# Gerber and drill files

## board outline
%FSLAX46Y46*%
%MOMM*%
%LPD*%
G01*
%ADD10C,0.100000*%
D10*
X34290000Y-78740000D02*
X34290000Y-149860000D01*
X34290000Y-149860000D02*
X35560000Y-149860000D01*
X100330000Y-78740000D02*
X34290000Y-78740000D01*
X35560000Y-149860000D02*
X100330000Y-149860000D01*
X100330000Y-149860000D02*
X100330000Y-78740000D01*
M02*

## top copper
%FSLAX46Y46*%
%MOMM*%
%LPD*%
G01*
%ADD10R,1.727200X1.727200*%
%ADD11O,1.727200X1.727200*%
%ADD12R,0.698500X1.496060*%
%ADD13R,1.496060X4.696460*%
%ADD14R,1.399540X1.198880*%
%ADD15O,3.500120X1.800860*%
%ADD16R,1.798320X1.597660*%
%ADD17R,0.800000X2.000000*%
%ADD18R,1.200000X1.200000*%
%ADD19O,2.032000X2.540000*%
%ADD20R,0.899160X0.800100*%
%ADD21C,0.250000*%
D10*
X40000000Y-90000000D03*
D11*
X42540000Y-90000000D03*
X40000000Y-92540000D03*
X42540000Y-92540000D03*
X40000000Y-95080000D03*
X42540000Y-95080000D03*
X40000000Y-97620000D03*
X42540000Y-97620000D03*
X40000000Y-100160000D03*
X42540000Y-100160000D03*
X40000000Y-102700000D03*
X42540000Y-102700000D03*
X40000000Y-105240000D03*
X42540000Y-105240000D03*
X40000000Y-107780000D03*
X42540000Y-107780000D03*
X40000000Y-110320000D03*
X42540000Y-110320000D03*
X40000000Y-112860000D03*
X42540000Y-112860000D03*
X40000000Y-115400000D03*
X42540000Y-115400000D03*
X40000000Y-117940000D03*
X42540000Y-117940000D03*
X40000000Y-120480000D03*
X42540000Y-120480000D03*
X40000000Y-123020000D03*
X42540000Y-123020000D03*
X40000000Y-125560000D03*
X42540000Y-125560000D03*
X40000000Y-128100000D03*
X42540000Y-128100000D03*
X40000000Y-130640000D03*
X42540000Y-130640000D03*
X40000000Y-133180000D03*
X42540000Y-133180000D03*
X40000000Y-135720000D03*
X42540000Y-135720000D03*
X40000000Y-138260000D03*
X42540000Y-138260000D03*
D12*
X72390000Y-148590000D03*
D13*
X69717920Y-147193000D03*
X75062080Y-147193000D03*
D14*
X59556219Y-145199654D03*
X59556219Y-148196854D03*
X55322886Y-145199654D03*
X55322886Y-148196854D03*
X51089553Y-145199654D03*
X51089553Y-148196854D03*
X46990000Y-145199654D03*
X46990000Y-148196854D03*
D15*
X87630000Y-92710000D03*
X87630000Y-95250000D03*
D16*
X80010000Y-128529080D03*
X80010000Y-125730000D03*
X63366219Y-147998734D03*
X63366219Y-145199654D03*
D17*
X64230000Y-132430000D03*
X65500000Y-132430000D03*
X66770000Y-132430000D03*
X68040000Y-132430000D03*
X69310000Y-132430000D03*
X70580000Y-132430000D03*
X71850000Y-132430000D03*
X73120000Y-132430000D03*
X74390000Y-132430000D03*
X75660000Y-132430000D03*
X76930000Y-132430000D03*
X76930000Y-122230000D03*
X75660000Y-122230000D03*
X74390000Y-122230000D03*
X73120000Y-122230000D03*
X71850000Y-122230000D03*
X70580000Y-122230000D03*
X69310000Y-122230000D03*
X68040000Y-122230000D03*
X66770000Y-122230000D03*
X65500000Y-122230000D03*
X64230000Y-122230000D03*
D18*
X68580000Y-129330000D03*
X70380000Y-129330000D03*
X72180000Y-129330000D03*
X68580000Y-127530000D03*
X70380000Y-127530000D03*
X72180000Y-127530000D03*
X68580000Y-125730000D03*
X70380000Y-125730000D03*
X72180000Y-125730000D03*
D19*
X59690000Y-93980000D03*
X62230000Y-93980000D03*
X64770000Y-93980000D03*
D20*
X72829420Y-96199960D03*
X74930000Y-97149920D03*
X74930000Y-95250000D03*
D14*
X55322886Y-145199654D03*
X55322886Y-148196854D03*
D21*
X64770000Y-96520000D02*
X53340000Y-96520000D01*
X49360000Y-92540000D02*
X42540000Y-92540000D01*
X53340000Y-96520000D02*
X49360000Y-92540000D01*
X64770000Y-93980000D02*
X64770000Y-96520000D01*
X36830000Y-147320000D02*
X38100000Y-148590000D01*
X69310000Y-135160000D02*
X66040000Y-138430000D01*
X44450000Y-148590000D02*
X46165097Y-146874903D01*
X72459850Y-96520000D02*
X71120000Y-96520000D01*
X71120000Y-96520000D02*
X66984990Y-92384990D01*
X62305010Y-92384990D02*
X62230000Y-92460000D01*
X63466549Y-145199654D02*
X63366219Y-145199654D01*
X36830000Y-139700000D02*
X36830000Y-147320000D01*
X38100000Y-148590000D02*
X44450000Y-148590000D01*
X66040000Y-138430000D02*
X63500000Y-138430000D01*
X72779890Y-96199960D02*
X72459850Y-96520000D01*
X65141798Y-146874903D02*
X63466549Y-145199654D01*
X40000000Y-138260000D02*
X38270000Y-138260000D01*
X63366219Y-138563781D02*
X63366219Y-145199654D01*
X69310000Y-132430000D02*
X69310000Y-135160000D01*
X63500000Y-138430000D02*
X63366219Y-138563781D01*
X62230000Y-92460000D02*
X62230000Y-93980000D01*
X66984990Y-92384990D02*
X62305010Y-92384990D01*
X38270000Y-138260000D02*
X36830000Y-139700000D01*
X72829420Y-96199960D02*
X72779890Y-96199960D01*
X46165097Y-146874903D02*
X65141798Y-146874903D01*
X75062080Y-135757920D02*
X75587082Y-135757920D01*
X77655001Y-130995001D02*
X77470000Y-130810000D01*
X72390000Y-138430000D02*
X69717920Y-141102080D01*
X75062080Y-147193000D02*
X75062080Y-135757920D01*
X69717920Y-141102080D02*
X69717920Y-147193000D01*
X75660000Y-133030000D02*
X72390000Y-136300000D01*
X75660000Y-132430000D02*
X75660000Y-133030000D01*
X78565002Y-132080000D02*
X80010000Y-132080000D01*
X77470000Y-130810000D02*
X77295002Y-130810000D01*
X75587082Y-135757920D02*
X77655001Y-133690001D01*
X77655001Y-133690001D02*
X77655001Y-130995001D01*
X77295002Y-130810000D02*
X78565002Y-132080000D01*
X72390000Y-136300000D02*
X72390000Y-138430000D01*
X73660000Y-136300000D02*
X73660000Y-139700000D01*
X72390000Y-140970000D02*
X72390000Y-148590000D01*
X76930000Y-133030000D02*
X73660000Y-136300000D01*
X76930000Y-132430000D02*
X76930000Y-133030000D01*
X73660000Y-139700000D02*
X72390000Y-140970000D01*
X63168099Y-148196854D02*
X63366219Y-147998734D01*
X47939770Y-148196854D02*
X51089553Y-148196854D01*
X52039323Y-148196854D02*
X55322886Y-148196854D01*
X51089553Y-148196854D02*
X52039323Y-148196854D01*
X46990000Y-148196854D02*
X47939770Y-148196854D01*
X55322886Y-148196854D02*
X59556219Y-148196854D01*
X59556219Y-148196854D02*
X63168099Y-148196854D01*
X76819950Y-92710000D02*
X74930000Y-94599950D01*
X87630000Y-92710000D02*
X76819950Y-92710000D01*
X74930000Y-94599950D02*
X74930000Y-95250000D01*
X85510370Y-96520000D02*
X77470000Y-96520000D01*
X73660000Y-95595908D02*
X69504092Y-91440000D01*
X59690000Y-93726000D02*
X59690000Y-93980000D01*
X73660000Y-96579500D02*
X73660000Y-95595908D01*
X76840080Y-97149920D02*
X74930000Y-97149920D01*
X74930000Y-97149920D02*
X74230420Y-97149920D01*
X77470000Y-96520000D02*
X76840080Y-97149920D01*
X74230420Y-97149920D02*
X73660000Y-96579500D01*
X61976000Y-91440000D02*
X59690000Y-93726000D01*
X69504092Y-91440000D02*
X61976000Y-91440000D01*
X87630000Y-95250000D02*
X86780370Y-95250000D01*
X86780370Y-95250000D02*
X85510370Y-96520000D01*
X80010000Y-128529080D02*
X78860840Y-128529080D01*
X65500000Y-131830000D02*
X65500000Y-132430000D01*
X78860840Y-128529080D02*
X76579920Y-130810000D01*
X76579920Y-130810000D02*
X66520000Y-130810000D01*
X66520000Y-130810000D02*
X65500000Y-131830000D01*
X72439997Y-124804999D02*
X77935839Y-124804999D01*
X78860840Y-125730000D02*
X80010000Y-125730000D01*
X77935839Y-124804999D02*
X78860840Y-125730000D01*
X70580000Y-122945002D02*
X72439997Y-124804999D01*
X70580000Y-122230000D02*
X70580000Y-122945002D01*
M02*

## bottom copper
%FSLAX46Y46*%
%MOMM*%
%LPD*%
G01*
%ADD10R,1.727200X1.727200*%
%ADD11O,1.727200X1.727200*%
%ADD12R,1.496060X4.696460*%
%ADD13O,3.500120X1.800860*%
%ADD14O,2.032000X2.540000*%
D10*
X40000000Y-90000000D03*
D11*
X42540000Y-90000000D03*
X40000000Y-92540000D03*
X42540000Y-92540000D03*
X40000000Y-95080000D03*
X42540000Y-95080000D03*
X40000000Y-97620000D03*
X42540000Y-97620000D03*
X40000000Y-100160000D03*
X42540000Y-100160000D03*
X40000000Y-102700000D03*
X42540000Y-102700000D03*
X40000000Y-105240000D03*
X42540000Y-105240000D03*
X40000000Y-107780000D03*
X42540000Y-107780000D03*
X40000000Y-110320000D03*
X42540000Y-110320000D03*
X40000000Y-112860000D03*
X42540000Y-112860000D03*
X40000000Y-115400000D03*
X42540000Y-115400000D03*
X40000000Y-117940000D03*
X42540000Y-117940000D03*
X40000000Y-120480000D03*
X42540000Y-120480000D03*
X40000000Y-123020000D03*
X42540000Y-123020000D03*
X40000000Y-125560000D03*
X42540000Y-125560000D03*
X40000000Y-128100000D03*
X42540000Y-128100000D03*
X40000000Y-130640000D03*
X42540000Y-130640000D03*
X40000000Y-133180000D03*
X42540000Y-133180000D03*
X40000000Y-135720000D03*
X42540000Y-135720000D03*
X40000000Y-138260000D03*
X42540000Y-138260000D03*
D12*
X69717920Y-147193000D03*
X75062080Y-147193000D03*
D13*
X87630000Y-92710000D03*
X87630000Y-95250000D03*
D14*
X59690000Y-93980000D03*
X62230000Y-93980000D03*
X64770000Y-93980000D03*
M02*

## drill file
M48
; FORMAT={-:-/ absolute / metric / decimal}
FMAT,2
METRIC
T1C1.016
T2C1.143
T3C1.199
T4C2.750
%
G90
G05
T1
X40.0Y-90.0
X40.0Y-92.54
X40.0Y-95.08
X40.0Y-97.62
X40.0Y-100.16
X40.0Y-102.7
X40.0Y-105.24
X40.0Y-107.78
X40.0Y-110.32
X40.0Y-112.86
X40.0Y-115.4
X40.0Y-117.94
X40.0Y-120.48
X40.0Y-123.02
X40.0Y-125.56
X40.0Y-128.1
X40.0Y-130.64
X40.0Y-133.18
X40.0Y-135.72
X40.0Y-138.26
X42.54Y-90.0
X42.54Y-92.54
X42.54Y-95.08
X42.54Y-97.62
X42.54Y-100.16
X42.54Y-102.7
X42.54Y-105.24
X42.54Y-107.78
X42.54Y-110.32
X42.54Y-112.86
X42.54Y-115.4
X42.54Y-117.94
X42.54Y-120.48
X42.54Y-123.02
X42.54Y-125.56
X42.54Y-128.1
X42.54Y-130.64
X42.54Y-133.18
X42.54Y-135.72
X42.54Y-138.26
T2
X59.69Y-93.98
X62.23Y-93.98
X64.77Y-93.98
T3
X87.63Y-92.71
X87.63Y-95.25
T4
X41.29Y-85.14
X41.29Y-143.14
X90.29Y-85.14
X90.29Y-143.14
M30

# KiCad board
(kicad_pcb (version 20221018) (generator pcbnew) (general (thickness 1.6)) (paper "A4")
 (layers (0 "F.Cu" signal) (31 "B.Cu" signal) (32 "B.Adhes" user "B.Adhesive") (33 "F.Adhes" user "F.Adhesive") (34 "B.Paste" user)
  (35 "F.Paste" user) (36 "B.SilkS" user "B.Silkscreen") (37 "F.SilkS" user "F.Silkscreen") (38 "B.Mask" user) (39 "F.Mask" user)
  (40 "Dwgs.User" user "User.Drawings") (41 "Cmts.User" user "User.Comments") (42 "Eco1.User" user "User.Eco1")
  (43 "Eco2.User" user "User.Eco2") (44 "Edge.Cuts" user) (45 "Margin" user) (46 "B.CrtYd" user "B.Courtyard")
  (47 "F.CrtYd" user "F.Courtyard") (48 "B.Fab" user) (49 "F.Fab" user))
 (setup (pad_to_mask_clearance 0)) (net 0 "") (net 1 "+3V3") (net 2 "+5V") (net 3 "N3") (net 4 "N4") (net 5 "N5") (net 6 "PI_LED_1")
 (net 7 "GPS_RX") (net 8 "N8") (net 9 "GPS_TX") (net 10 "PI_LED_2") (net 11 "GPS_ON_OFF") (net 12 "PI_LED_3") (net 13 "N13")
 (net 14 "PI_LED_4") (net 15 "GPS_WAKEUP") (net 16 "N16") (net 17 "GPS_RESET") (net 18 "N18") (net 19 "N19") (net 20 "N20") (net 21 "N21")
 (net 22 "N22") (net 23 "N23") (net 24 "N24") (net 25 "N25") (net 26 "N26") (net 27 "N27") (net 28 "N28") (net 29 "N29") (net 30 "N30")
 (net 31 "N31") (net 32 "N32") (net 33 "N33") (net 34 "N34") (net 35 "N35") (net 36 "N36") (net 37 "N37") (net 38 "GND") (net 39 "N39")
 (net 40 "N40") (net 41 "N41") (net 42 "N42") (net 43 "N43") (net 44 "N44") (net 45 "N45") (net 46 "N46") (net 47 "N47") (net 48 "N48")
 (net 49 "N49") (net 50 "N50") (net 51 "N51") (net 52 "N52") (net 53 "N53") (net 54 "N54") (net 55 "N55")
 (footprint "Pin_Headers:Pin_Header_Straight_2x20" (layer "F.Cu") (at 40 90)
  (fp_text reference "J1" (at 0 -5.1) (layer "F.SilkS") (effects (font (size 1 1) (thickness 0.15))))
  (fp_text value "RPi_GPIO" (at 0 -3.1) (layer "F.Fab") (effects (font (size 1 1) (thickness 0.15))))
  (pad "1" thru_hole rect (at 0 0) (size 1.7272 1.7272) (drill 1.016) (layers "*.Cu" "*.Mask" "F.SilkS") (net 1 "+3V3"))
  (pad "2" thru_hole oval (at 2.54 0) (size 1.7272 1.7272) (drill 1.016) (layers "*.Cu" "*.Mask" "F.SilkS") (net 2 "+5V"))
  (pad "3" thru_hole oval (at 0 2.54) (size 1.7272 1.7272) (drill 1.016) (layers "*.Cu" "*.Mask" "F.SilkS") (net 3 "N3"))
  (pad "4" thru_hole oval (at 2.54 2.54) (size 1.7272 1.7272) (drill 1.016) (layers "*.Cu" "*.Mask" "F.SilkS") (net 2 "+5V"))
  (pad "5" thru_hole oval (at 0 5.08) (size 1.7272 1.7272) (drill 1.016) (layers "*.Cu" "*.Mask" "F.SilkS") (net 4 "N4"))
  (pad "6" thru_hole oval (at 2.54 5.08) (size 1.7272 1.7272) (drill 1.016) (layers "*.Cu" "*.Mask" "F.SilkS") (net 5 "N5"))
  (pad "7" thru_hole oval (at 0 7.62) (size 1.7272 1.7272) (drill 1.016) (layers "*.Cu" "*.Mask" "F.SilkS") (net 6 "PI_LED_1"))
  (pad "8" thru_hole oval (at 2.54 7.62) (size 1.7272 1.7272) (drill 1.016) (layers "*.Cu" "*.Mask" "F.SilkS") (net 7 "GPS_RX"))
  (pad "9" thru_hole oval (at 0 10.16) (size 1.7272 1.7272) (drill 1.016) (layers "*.Cu" "*.Mask" "F.SilkS") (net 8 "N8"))
  (pad "10" thru_hole oval (at 2.54 10.16) (size 1.7272 1.7272) (drill 1.016) (layers "*.Cu" "*.Mask" "F.SilkS") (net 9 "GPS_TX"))
  (pad "11" thru_hole oval (at 0 12.7) (size 1.7272 1.7272) (drill 1.016) (layers "*.Cu" "*.Mask" "F.SilkS") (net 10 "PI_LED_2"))
  (pad "12" thru_hole oval (at 2.54 12.7) (size 1.7272 1.7272) (drill 1.016) (layers "*.Cu" "*.Mask" "F.SilkS") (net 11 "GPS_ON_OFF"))
  (pad "13" thru_hole oval (at 0 15.24) (size 1.7272 1.7272) (drill 1.016) (layers "*.Cu" "*.Mask" "F.SilkS") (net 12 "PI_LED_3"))
  (pad "14" thru_hole oval (at 2.54 15.24) (size 1.7272 1.7272) (drill 1.016) (layers "*.Cu" "*.Mask" "F.SilkS") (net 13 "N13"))
  (pad "15" thru_hole oval (at 0 17.78) (size 1.7272 1.7272) (drill 1.016) (layers "*.Cu" "*.Mask" "F.SilkS") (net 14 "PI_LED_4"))
  (pad "16" thru_hole oval (at 2.54 17.78) (size 1.7272 1.7272) (drill 1.016) (layers "*.Cu" "*.Mask" "F.SilkS") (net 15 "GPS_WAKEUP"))
  (pad "17" thru_hole oval (at 0 20.32) (size 1.7272 1.7272) (drill 1.016) (layers "*.Cu" "*.Mask" "F.SilkS") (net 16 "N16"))
  (pad "18" thru_hole oval (at 2.54 20.32) (size 1.7272 1.7272) (drill 1.016) (layers "*.Cu" "*.Mask" "F.SilkS") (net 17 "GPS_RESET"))
  (pad "19" thru_hole oval (at 0 22.86) (size 1.7272 1.7272) (drill 1.016) (layers "*.Cu" "*.Mask" "F.SilkS") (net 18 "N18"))
  (pad "20" thru_hole oval (at 2.54 22.86) (size 1.7272 1.7272) (drill 1.016) (layers "*.Cu" "*.Mask" "F.SilkS") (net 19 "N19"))
  (pad "21" thru_hole oval (at 0 25.4) (size 1.7272 1.7272) (drill 1.016) (layers "*.Cu" "*.Mask" "F.SilkS") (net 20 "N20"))
  (pad "22" thru_hole oval (at 2.54 25.4) (size 1.7272 1.7272) (drill 1.016) (layers "*.Cu" "*.Mask" "F.SilkS") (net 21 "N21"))
  (pad "23" thru_hole oval (at 0 27.94) (size 1.7272 1.7272) (drill 1.016) (layers "*.Cu" "*.Mask" "F.SilkS") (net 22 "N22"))
  (pad "24" thru_hole oval (at 2.54 27.94) (size 1.7272 1.7272) (drill 1.016) (layers "*.Cu" "*.Mask" "F.SilkS") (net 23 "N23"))
  (pad "25" thru_hole oval (at 0 30.48) (size 1.7272 1.7272) (drill 1.016) (layers "*.Cu" "*.Mask" "F.SilkS") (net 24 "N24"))
  (pad "26" thru_hole oval (at 2.54 30.48) (size 1.7272 1.7272) (drill 1.016) (layers "*.Cu" "*.Mask" "F.SilkS") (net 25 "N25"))
  (pad "27" thru_hole oval (at 0 33.02) (size 1.7272 1.7272) (drill 1.016) (layers "*.Cu" "*.Mask" "F.SilkS") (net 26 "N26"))
  (pad "28" thru_hole oval (at 2.54 33.02) (size 1.7272 1.7272) (drill 1.016) (layers "*.Cu" "*.Mask" "F.SilkS") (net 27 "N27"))
  (pad "29" thru_hole oval (at 0 35.56) (size 1.7272 1.7272) (drill 1.016) (layers "*.Cu" "*.Mask" "F.SilkS") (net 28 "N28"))
  (pad "30" thru_hole oval (at 2.54 35.56) (size 1.7272 1.7272) (drill 1.016) (layers "*.Cu" "*.Mask" "F.SilkS") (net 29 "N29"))
  (pad "31" thru_hole oval (at 0 38.1) (size 1.7272 1.7272) (drill 1.016) (layers "*.Cu" "*.Mask" "F.SilkS") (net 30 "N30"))
  (pad "32" thru_hole oval (at 2.54 38.1) (size 1.7272 1.7272) (drill 1.016) (layers "*.Cu" "*.Mask" "F.SilkS") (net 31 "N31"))
  (pad "33" thru_hole oval (at 0 40.64) (size 1.7272 1.7272) (drill 1.016) (layers "*.Cu" "*.Mask" "F.SilkS") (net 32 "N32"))
  (pad "34" thru_hole oval (at 2.54 40.64) (size 1.7272 1.7272) (drill 1.016) (layers "*.Cu" "*.Mask" "F.SilkS") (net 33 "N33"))
  (pad "35" thru_hole oval (at 0 43.18) (size 1.7272 1.7272) (drill 1.016) (layers "*.Cu" "*.Mask" "F.SilkS") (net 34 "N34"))
  (pad "36" thru_hole oval (at 2.54 43.18) (size 1.7272 1.7272) (drill 1.016) (layers "*.Cu" "*.Mask" "F.SilkS") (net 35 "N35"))
  (pad "37" thru_hole oval (at 0 45.72) (size 1.7272 1.7272) (drill 1.016) (layers "*.Cu" "*.Mask" "F.SilkS") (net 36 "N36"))
  (pad "38" thru_hole oval (at 2.54 45.72) (size 1.7272 1.7272) (drill 1.016) (layers "*.Cu" "*.Mask" "F.SilkS") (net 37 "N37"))
  (pad "39" thru_hole oval (at 0 48.26) (size 1.7272 1.7272) (drill 1.016) (layers "*.Cu" "*.Mask" "F.SilkS") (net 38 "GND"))
  (pad "40" thru_hole oval (at 2.54 48.26) (size 1.7272 1.7272) (drill 1.016) (layers "*.Cu" "*.Mask" "F.SilkS") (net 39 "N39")))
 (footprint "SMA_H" (layer "F.Cu") (at 72.39 147.193 -90)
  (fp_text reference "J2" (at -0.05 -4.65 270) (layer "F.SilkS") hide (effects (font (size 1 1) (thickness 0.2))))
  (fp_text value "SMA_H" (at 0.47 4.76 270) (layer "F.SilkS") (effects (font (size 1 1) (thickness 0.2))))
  (pad "1" smd rect (at 1.397 0 270) (size 1.49606 0.6985) (layers "F.Cu" "F.Paste" "F.Mask") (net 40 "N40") (clearance 0.19558))
  (pad "2" smd rect (at 0 2.67208 270) (size 4.69646 1.49606) (layers "F.Cu" "F.Paste" "F.Mask") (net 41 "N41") (clearance 0.19558))
  (pad "3" smd rect (at 0 -2.67208 270) (size 4.69646 1.49606) (layers "F.Cu" "F.Paste" "F.Mask") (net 41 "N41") (clearance 0.19558))
  (pad "4" smd rect (at 0 2.67208 270) (size 4.69646 1.49606) (layers "B.Cu" "B.Paste" "B.Mask") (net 41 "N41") (clearance 0.19558))
  (pad "5" smd rect (at 0 -2.67208 270) (size 4.69646 1.49606) (layers "B.Cu" "B.Paste" "B.Mask") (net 41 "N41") (clearance 0.19558)))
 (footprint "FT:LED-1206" (layer "F.Cu") (at 59.556219 146.698254 -90)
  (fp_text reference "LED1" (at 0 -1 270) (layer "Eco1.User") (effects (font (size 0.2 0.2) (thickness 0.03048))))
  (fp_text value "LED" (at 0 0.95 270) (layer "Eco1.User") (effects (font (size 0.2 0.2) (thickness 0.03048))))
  (pad "A" smd rect (at -1.4986 0 270) (size 1.19888 1.39954) (layers "F.Cu" "F.Paste" "F.Mask") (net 6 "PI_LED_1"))
  (pad "K" smd rect (at 1.4986 0 270) (size 1.19888 1.39954) (layers "F.Cu" "F.Paste" "F.Mask") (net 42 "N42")))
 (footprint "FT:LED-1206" (layer "F.Cu") (at 55.322886 146.698254 -90)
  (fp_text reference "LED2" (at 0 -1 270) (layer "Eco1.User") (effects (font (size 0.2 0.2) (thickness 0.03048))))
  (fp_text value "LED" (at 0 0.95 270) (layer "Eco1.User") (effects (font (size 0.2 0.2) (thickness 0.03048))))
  (pad "A" smd rect (at -1.4986 0 270) (size 1.19888 1.39954) (layers "F.Cu" "F.Paste" "F.Mask") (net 10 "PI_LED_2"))
  (pad "K" smd rect (at 1.4986 0 270) (size 1.19888 1.39954) (layers "F.Cu" "F.Paste" "F.Mask") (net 42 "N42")))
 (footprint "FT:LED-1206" (layer "F.Cu") (at 51.089553 146.698254 -90)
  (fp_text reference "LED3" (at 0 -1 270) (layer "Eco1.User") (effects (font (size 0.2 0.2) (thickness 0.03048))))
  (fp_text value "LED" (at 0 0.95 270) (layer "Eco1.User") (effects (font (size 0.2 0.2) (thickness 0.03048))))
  (pad "A" smd rect (at -1.4986 0 270) (size 1.19888 1.39954) (layers "F.Cu" "F.Paste" "F.Mask") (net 12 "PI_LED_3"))
  (pad "K" smd rect (at 1.4986 0 270) (size 1.19888 1.39954) (layers "F.Cu" "F.Paste" "F.Mask") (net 42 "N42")))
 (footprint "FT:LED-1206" (layer "F.Cu") (at 46.99 146.698254 -90)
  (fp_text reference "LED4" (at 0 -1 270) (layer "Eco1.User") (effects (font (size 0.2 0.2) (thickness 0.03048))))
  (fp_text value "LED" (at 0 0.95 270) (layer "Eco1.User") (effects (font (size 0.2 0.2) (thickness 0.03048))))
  (pad "A" smd rect (at -1.4986 0 270) (size 1.19888 1.39954) (layers "F.Cu" "F.Paste" "F.Mask") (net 14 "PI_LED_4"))
  (pad "K" smd rect (at 1.4986 0 270) (size 1.19888 1.39954) (layers "F.Cu" "F.Paste" "F.Mask") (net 42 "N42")))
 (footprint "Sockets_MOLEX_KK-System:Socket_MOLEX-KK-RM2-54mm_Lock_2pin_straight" (layer "F.Cu") (at 87.63 93.98 -90)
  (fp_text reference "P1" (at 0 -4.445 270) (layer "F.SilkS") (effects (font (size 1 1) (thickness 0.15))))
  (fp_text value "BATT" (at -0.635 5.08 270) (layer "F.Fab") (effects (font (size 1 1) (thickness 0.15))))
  (pad "1" thru_hole oval (at -1.27 0 270) (size 1.80086 3.50012) (drill 1.19888) (layers "*.Cu" "*.Mask" "F.SilkS") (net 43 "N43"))
  (pad "2" thru_hole oval (at 1.27 0 270) (size 1.80086 3.50012) (drill 1.19888) (layers "*.Cu" "*.Mask" "F.SilkS") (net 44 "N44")))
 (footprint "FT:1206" (layer "F.Cu") (at 80.01 127.12954 90)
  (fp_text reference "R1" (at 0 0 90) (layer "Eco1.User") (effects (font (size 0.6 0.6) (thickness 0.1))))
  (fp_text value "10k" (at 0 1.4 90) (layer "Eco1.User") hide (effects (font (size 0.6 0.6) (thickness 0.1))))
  (pad "1" smd rect (at -1.39954 0 90) (size 1.59766 1.79832) (layers "F.Cu" "F.Paste" "F.Mask") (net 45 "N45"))
  (pad "2" smd rect (at 1.39954 0 90) (size 1.59766 1.79832) (layers "F.Cu" "F.Paste" "F.Mask") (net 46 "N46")))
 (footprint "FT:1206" (layer "F.Cu") (at 63.366219 146.599194 90)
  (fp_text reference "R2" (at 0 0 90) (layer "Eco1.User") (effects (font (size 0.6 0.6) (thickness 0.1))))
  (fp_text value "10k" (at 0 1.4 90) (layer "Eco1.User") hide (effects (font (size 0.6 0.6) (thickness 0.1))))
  (pad "1" smd rect (at -1.39954 0 90) (size 1.59766 1.79832) (layers "F.Cu" "F.Paste" "F.Mask") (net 42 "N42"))
  (pad "2" smd rect (at 1.39954 0 90) (size 1.59766 1.79832) (layers "F.Cu" "F.Paste" "F.Mask") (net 38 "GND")))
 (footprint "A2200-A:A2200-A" (layer "F.Cu") (at 70.38 127.53 90)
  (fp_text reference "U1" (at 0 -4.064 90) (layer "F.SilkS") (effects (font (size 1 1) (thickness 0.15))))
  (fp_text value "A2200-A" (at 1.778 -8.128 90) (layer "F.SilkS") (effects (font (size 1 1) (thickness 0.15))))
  (pad "1" smd rect (at -4.9 -6.15 90) (size 2 0.8) (layers "F.Cu" "F.Paste" "F.Mask") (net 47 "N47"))
  (pad "2" smd rect (at -4.9 -4.88 90) (size 2 0.8) (layers "F.Cu" "F.Paste" "F.Mask") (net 45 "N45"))
  (pad "3" smd rect (at -4.9 -3.61 90) (size 2 0.8) (layers "F.Cu" "F.Paste" "F.Mask") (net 9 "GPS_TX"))
  (pad "4" smd rect (at -4.9 -2.34 90) (size 2 0.8) (layers "F.Cu" "F.Paste" "F.Mask") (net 7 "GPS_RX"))
  (pad "5" smd rect (at -4.9 -1.07 90) (size 2 0.8) (layers "F.Cu" "F.Paste" "F.Mask") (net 38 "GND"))
  (pad "6" smd rect (at -4.9 0.2 90) (size 2 0.8) (layers "F.Cu" "F.Paste" "F.Mask") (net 11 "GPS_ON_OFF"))
  (pad "7" smd rect (at -4.9 1.47 90) (size 2 0.8) (layers "F.Cu" "F.Paste" "F.Mask") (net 38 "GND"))
  (pad "8" smd rect (at -4.9 2.74 90) (size 2 0.8) (layers "F.Cu" "F.Paste" "F.Mask") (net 38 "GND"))
  (pad "9" smd rect (at -4.9 4.01 90) (size 2 0.8) (layers "F.Cu" "F.Paste" "F.Mask") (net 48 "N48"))
  (pad "10" smd rect (at -4.9 5.28 90) (size 2 0.8) (layers "F.Cu" "F.Paste" "F.Mask") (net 41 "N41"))
  (pad "11" smd rect (at -4.9 6.55 90) (size 2 0.8) (layers "F.Cu" "F.Paste" "F.Mask") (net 40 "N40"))
  (pad "12" smd rect (at 5.3 6.55 90) (size 2 0.8) (layers "F.Cu" "F.Paste" "F.Mask") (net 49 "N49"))
  (pad "13" smd rect (at 5.3 5.28 90) (size 2 0.8) (layers "F.Cu" "F.Paste" "F.Mask") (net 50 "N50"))
  (pad "14" smd rect (at 5.3 4.01 90) (size 2 0.8) (layers "F.Cu" "F.Paste" "F.Mask") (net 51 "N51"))
  (pad "15" smd rect (at 5.3 2.74 90) (size 2 0.8) (layers "F.Cu" "F.Paste" "F.Mask") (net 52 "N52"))
  (pad "16" smd rect (at 5.3 1.47 90) (size 2 0.8) (layers "F.Cu" "F.Paste" "F.Mask") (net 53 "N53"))
  (pad "17" smd rect (at 5.3 0.2 90) (size 2 0.8) (layers "F.Cu" "F.Paste" "F.Mask") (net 46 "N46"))
  (pad "18" smd rect (at 5.3 -1.07 90) (size 2 0.8) (layers "F.Cu" "F.Paste" "F.Mask") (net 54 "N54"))
  (pad "19" smd rect (at 5.3 -2.34 90) (size 2 0.8) (layers "F.Cu" "F.Paste" "F.Mask") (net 15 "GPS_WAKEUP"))
  (pad "20" smd rect (at 5.3 -3.61 90) (size 2 0.8) (layers "F.Cu" "F.Paste" "F.Mask") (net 1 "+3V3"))
  (pad "21" smd rect (at 5.3 -4.88 90) (size 2 0.8) (layers "F.Cu" "F.Paste" "F.Mask") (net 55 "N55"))
  (pad "22" smd rect (at 5.3 -6.15 90) (size 2 0.8) (layers "F.Cu" "F.Paste" "F.Mask") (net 17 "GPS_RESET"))
  (pad "23" smd rect (at -1.8 -1.8 90) (size 1.2 1.2) (layers "F.Cu" "F.Paste" "F.Mask"))
  (pad "24" smd rect (at -1.8 0 90) (size 1.2 1.2) (layers "F.Cu" "F.Paste" "F.Mask"))
  (pad "25" smd rect (at -1.8 1.8 90) (size 1.2 1.2) (layers "F.Cu" "F.Paste" "F.Mask"))
  (pad "26" smd rect (at 0 -1.8 90) (size 1.2 1.2) (layers "F.Cu" "F.Paste" "F.Mask"))
  (pad "27" smd rect (at 0 0 90) (size 1.2 1.2) (layers "F.Cu" "F.Paste" "F.Mask"))
  (pad "29" smd rect (at 0 1.8 90) (size 1.2 1.2) (layers "F.Cu" "F.Paste" "F.Mask"))
  (pad "30" smd rect (at 1.8 -1.8 90) (size 1.2 1.2) (layers "F.Cu" "F.Paste" "F.Mask"))
  (pad "31" smd rect (at 1.8 0 90) (size 1.2 1.2) (layers "F.Cu" "F.Paste" "F.Mask"))
  (pad "32" smd rect (at 1.8 1.8 90) (size 1.2 1.2) (layers "F.Cu" "F.Paste" "F.Mask")))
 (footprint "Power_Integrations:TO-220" (layer "F.Cu") (at 62.23 93.98)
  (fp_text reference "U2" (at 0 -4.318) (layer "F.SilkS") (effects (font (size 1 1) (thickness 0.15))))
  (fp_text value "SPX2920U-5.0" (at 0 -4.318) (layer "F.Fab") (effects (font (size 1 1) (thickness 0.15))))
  (pad "1" thru_hole oval (at -2.54 0) (size 2.032 2.54) (drill 1.143) (layers "*.Cu" "*.Mask" "F.SilkS") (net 44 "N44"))
  (pad "2" thru_hole oval (at 0 0) (size 2.032 2.54) (drill 1.143) (layers "*.Cu" "*.Mask" "F.SilkS") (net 38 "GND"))
  (pad "3" thru_hole oval (at 2.54 0) (size 2.032 2.54) (drill 1.143) (layers "*.Cu" "*.Mask" "F.SilkS") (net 2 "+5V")))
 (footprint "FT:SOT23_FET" (layer "F.Cu") (at 73.92924 96.19996 90)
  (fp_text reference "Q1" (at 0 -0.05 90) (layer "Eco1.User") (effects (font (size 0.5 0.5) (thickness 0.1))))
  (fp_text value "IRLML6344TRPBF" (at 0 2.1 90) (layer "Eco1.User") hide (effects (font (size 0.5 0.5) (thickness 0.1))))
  (pad "D" smd rect (at 0 -1.09982 90) (size 0.8001 0.89916) (layers "F.Cu" "F.Paste" "F.Mask") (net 38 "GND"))
  (pad "G" smd rect (at -0.94996 1.00076 90) (size 0.8001 0.89916) (layers "F.Cu" "F.Paste" "F.Mask") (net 44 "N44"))
  (pad "S" smd rect (at 0.94996 1.00076 90) (size 0.8001 0.89916) (layers "F.Cu" "F.Paste" "F.Mask") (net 43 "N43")))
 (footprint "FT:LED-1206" (layer "F.Cu") (at 55.322886 146.698254 -90)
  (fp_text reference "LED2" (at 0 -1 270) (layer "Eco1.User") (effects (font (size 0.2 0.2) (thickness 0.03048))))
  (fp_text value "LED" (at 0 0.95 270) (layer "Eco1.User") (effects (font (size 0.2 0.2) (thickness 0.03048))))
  (pad "A" smd rect (at -1.4986 0 270) (size 1.19888 1.39954) (layers "F.Cu" "F.Paste" "F.Mask") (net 10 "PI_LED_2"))
  (pad "K" smd rect (at 1.4986 0 270) (size 1.19888 1.39954) (layers "F.Cu" "F.Paste" "F.Mask") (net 42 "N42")))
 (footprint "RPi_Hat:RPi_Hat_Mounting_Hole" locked (layer "F.Cu") (at 41.29 143.14)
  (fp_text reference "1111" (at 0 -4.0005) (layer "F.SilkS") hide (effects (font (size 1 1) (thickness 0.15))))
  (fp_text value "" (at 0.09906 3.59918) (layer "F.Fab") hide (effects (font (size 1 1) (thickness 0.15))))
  (pad "" np_thru_hole circle locked (at 0 0) (size 2.75 2.75) (drill 2.75) (layers "*.Cu" "*.Mask") (solder_mask_margin 1.725)
   (clearance 1.725)))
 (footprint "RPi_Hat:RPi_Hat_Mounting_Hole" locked (layer "F.Cu") (at 90.29 143.14)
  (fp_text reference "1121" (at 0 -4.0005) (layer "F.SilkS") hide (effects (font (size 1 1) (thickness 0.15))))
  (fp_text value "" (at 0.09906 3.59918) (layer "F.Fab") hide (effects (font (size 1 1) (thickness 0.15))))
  (pad "" np_thru_hole circle locked (at 0 0) (size 2.75 2.75) (drill 2.75) (layers "*.Cu" "*.Mask") (solder_mask_margin 1.725)
   (clearance 1.725)))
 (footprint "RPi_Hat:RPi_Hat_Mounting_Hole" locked (layer "F.Cu") (at 41.29 85.14)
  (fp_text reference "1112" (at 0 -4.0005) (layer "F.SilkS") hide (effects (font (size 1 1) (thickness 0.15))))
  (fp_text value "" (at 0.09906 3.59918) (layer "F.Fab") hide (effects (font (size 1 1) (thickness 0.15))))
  (pad "" np_thru_hole circle locked (at 0 0) (size 2.75 2.75) (drill 2.75) (layers "*.Cu" "*.Mask") (solder_mask_margin 1.725)
   (clearance 1.725)))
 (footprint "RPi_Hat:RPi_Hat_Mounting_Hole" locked (layer "F.Cu") (at 90.29 85.14)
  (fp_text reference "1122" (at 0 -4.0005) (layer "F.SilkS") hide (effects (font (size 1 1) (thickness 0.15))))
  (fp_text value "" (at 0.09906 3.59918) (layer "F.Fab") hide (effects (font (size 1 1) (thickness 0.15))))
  (pad "" np_thru_hole circle locked (at 0 0) (size 2.75 2.75) (drill 2.75) (layers "*.Cu" "*.Mask") (solder_mask_margin 1.725)
   (clearance 1.725)))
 (gr_line (start 34.29 78.74) (end 34.29 149.86) (stroke (width 0.1) (type solid)) (layer "Edge.Cuts"))
 (gr_line (start 34.29 149.86) (end 35.56 149.86) (stroke (width 0.1) (type solid)) (layer "Edge.Cuts"))
 (gr_line (start 100.33 78.74) (end 34.29 78.74) (stroke (width 0.1) (type solid)) (layer "Edge.Cuts"))
 (gr_line (start 35.56 149.86) (end 100.33 149.86) (stroke (width 0.1) (type solid)) (layer "Edge.Cuts"))
 (gr_line (start 100.33 149.86) (end 100.33 78.74) (stroke (width 0.1) (type solid)) (layer "Edge.Cuts"))
 (segment (start 64.77 96.52) (end 53.34 96.52) (width 0.25) (layer "F.Cu") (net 2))
 (segment (start 49.36 92.54) (end 42.54 92.54) (width 0.25) (layer "F.Cu") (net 2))
 (segment (start 53.34 96.52) (end 49.36 92.54) (width 0.25) (layer "F.Cu") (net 2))
 (segment (start 64.77 93.98) (end 64.77 96.52) (width 0.25) (layer "F.Cu") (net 2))
 (segment (start 36.83 147.32) (end 38.1 148.59) (width 0.25) (layer "F.Cu") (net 38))
 (segment (start 69.31 135.16) (end 66.04 138.43) (width 0.25) (layer "F.Cu") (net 38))
 (segment (start 44.45 148.59) (end 46.165097 146.874903) (width 0.25) (layer "F.Cu") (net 38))
 (segment (start 72.45985 96.52) (end 71.12 96.52) (width 0.25) (layer "F.Cu") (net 38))
 (segment (start 71.12 96.52) (end 66.98499 92.38499) (width 0.25) (layer "F.Cu") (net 38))
 (segment (start 62.30501 92.38499) (end 62.23 92.46) (width 0.25) (layer "F.Cu") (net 38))
 (segment (start 63.466549 145.199654) (end 63.366219 145.199654) (width 0.25) (layer "F.Cu") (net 38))
 (segment (start 36.83 139.7) (end 36.83 147.32) (width 0.25) (layer "F.Cu") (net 38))
 (segment (start 38.1 148.59) (end 44.45 148.59) (width 0.25) (layer "F.Cu") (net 38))
 (segment (start 66.04 138.43) (end 63.5 138.43) (width 0.25) (layer "F.Cu") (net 38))
 (segment (start 72.77989 96.19996) (end 72.45985 96.52) (width 0.25) (layer "F.Cu") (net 38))
 (segment (start 65.141798 146.874903) (end 63.466549 145.199654) (width 0.25) (layer "F.Cu") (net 38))
 (segment (start 40 138.26) (end 38.27 138.26) (width 0.25) (layer "F.Cu") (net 38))
 (segment (start 63.366219 138.563781) (end 63.366219 145.199654) (width 0.25) (layer "F.Cu") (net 38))
 (segment (start 69.31 132.43) (end 69.31 135.16) (width 0.25) (layer "F.Cu") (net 38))
 (segment (start 63.5 138.43) (end 63.366219 138.563781) (width 0.25) (layer "F.Cu") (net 38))
 (segment (start 62.23 92.46) (end 62.23 93.98) (width 0.25) (layer "F.Cu") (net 38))
 (segment (start 66.98499 92.38499) (end 62.30501 92.38499) (width 0.25) (layer "F.Cu") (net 38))
 (segment (start 38.27 138.26) (end 36.83 139.7) (width 0.25) (layer "F.Cu") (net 38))
 (segment (start 72.82942 96.19996) (end 72.77989 96.19996) (width 0.25) (layer "F.Cu") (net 38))
 (segment (start 46.165097 146.874903) (end 65.141798 146.874903) (width 0.25) (layer "F.Cu") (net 38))
 (segment (start 75.06208 135.75792) (end 75.587082 135.75792) (width 0.25) (layer "F.Cu") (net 41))
 (segment (start 77.655001 130.995001) (end 77.47 130.81) (width 0.25) (layer "F.Cu") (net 41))
 (segment (start 72.39 138.43) (end 69.71792 141.10208) (width 0.25) (layer "F.Cu") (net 41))
 (segment (start 75.06208 147.193) (end 75.06208 135.75792) (width 0.25) (layer "F.Cu") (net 41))
 (segment (start 69.71792 141.10208) (end 69.71792 147.193) (width 0.25) (layer "F.Cu") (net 41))
 (segment (start 75.66 133.03) (end 72.39 136.3) (width 0.25) (layer "F.Cu") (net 41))
 (segment (start 75.66 132.43) (end 75.66 133.03) (width 0.25) (layer "F.Cu") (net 41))
 (segment (start 78.565002 132.08) (end 80.01 132.08) (width 0.25) (layer "F.Cu") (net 41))
 (segment (start 77.47 130.81) (end 77.295002 130.81) (width 0.25) (layer "F.Cu") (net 41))
 (segment (start 75.587082 135.75792) (end 77.655001 133.690001) (width 0.25) (layer "F.Cu") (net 41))
 (segment (start 77.655001 133.690001) (end 77.655001 130.995001) (width 0.25) (layer "F.Cu") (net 41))
 (segment (start 77.295002 130.81) (end 78.565002 132.08) (width 0.25) (layer "F.Cu") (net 41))
 (segment (start 72.39 136.3) (end 72.39 138.43) (width 0.25) (layer "F.Cu") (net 41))
 (segment (start 73.66 136.3) (end 73.66 139.7) (width 0.25) (layer "F.Cu") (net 40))
 (segment (start 72.39 140.97) (end 72.39 148.59) (width 0.25) (layer "F.Cu") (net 40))
 (segment (start 76.93 133.03) (end 73.66 136.3) (width 0.25) (layer "F.Cu") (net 40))
 (segment (start 76.93 132.43) (end 76.93 133.03) (width 0.25) (layer "F.Cu") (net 40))
 (segment (start 73.66 139.7) (end 72.39 140.97) (width 0.25) (layer "F.Cu") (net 40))
 (segment (start 63.168099 148.196854) (end 63.366219 147.998734) (width 0.25) (layer "F.Cu") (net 42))
 (segment (start 47.93977 148.196854) (end 51.089553 148.196854) (width 0.25) (layer "F.Cu") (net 42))
 (segment (start 52.039323 148.196854) (end 55.322886 148.196854) (width 0.25) (layer "F.Cu") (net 42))
 (segment (start 51.089553 148.196854) (end 52.039323 148.196854) (width 0.25) (layer "F.Cu") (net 42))
 (segment (start 46.99 148.196854) (end 47.93977 148.196854) (width 0.25) (layer "F.Cu") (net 42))
 (segment (start 55.322886 148.196854) (end 59.556219 148.196854) (width 0.25) (layer "F.Cu") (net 42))
 (segment (start 59.556219 148.196854) (end 63.168099 148.196854) (width 0.25) (layer "F.Cu") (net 42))
 (segment (start 76.81995 92.71) (end 74.93 94.59995) (width 0.25) (layer "F.Cu") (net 43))
 (segment (start 87.63 92.71) (end 76.81995 92.71) (width 0.25) (layer "F.Cu") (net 43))
 (segment (start 74.93 94.59995) (end 74.93 95.25) (width 0.25) (layer "F.Cu") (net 43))
 (segment (start 85.51037 96.52) (end 77.47 96.52) (width 0.25) (layer "F.Cu") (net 44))
 (segment (start 73.66 95.595908) (end 69.504092 91.44) (width 0.25) (layer "F.Cu") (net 44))
 (segment (start 59.69 93.726) (end 59.69 93.98) (width 0.25) (layer "F.Cu") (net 44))
 (segment (start 73.66 96.5795) (end 73.66 95.595908) (width 0.25) (layer "F.Cu") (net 44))
 (segment (start 76.84008 97.14992) (end 74.93 97.14992) (width 0.25) (layer "F.Cu") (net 44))
 (segment (start 74.93 97.14992) (end 74.23042 97.14992) (width 0.25) (layer "F.Cu") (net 44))
 (segment (start 77.47 96.52) (end 76.84008 97.14992) (width 0.25) (layer "F.Cu") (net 44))
 (segment (start 74.23042 97.14992) (end 73.66 96.5795) (width 0.25) (layer "F.Cu") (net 44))
 (segment (start 61.976 91.44) (end 59.69 93.726) (width 0.25) (layer "F.Cu") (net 44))
 (segment (start 69.504092 91.44) (end 61.976 91.44) (width 0.25) (layer "F.Cu") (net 44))
 (segment (start 87.63 95.25) (end 86.78037 95.25) (width 0.25) (layer "F.Cu") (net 44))
 (segment (start 86.78037 95.25) (end 85.51037 96.52) (width 0.25) (layer "F.Cu") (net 44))
 (segment (start 80.01 128.52908) (end 78.86084 128.52908) (width 0.25) (layer "F.Cu") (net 45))
 (segment (start 65.5 131.83) (end 65.5 132.43) (width 0.25) (layer "F.Cu") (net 45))
 (segment (start 78.86084 128.52908) (end 76.57992 130.81) (width 0.25) (layer "F.Cu") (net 45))
 (segment (start 76.57992 130.81) (end 66.52 130.81) (width 0.25) (layer "F.Cu") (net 45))
 (segment (start 66.52 130.81) (end 65.5 131.83) (width 0.25) (layer "F.Cu") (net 45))
 (segment (start 72.439997 124.804999) (end 77.935839 124.804999) (width 0.25) (layer "F.Cu") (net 46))
 (segment (start 78.86084 125.73) (end 80.01 125.73) (width 0.25) (layer "F.Cu") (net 46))
 (segment (start 77.935839 124.804999) (end 78.86084 125.73) (width 0.25) (layer "F.Cu") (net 46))
 (segment (start 70.58 122.945002) (end 72.439997 124.804999) (width 0.25) (layer "F.Cu") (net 46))
 (segment (start 70.58 122.23) (end 70.58 122.945002) (width 0.25) (layer "F.Cu") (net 46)))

